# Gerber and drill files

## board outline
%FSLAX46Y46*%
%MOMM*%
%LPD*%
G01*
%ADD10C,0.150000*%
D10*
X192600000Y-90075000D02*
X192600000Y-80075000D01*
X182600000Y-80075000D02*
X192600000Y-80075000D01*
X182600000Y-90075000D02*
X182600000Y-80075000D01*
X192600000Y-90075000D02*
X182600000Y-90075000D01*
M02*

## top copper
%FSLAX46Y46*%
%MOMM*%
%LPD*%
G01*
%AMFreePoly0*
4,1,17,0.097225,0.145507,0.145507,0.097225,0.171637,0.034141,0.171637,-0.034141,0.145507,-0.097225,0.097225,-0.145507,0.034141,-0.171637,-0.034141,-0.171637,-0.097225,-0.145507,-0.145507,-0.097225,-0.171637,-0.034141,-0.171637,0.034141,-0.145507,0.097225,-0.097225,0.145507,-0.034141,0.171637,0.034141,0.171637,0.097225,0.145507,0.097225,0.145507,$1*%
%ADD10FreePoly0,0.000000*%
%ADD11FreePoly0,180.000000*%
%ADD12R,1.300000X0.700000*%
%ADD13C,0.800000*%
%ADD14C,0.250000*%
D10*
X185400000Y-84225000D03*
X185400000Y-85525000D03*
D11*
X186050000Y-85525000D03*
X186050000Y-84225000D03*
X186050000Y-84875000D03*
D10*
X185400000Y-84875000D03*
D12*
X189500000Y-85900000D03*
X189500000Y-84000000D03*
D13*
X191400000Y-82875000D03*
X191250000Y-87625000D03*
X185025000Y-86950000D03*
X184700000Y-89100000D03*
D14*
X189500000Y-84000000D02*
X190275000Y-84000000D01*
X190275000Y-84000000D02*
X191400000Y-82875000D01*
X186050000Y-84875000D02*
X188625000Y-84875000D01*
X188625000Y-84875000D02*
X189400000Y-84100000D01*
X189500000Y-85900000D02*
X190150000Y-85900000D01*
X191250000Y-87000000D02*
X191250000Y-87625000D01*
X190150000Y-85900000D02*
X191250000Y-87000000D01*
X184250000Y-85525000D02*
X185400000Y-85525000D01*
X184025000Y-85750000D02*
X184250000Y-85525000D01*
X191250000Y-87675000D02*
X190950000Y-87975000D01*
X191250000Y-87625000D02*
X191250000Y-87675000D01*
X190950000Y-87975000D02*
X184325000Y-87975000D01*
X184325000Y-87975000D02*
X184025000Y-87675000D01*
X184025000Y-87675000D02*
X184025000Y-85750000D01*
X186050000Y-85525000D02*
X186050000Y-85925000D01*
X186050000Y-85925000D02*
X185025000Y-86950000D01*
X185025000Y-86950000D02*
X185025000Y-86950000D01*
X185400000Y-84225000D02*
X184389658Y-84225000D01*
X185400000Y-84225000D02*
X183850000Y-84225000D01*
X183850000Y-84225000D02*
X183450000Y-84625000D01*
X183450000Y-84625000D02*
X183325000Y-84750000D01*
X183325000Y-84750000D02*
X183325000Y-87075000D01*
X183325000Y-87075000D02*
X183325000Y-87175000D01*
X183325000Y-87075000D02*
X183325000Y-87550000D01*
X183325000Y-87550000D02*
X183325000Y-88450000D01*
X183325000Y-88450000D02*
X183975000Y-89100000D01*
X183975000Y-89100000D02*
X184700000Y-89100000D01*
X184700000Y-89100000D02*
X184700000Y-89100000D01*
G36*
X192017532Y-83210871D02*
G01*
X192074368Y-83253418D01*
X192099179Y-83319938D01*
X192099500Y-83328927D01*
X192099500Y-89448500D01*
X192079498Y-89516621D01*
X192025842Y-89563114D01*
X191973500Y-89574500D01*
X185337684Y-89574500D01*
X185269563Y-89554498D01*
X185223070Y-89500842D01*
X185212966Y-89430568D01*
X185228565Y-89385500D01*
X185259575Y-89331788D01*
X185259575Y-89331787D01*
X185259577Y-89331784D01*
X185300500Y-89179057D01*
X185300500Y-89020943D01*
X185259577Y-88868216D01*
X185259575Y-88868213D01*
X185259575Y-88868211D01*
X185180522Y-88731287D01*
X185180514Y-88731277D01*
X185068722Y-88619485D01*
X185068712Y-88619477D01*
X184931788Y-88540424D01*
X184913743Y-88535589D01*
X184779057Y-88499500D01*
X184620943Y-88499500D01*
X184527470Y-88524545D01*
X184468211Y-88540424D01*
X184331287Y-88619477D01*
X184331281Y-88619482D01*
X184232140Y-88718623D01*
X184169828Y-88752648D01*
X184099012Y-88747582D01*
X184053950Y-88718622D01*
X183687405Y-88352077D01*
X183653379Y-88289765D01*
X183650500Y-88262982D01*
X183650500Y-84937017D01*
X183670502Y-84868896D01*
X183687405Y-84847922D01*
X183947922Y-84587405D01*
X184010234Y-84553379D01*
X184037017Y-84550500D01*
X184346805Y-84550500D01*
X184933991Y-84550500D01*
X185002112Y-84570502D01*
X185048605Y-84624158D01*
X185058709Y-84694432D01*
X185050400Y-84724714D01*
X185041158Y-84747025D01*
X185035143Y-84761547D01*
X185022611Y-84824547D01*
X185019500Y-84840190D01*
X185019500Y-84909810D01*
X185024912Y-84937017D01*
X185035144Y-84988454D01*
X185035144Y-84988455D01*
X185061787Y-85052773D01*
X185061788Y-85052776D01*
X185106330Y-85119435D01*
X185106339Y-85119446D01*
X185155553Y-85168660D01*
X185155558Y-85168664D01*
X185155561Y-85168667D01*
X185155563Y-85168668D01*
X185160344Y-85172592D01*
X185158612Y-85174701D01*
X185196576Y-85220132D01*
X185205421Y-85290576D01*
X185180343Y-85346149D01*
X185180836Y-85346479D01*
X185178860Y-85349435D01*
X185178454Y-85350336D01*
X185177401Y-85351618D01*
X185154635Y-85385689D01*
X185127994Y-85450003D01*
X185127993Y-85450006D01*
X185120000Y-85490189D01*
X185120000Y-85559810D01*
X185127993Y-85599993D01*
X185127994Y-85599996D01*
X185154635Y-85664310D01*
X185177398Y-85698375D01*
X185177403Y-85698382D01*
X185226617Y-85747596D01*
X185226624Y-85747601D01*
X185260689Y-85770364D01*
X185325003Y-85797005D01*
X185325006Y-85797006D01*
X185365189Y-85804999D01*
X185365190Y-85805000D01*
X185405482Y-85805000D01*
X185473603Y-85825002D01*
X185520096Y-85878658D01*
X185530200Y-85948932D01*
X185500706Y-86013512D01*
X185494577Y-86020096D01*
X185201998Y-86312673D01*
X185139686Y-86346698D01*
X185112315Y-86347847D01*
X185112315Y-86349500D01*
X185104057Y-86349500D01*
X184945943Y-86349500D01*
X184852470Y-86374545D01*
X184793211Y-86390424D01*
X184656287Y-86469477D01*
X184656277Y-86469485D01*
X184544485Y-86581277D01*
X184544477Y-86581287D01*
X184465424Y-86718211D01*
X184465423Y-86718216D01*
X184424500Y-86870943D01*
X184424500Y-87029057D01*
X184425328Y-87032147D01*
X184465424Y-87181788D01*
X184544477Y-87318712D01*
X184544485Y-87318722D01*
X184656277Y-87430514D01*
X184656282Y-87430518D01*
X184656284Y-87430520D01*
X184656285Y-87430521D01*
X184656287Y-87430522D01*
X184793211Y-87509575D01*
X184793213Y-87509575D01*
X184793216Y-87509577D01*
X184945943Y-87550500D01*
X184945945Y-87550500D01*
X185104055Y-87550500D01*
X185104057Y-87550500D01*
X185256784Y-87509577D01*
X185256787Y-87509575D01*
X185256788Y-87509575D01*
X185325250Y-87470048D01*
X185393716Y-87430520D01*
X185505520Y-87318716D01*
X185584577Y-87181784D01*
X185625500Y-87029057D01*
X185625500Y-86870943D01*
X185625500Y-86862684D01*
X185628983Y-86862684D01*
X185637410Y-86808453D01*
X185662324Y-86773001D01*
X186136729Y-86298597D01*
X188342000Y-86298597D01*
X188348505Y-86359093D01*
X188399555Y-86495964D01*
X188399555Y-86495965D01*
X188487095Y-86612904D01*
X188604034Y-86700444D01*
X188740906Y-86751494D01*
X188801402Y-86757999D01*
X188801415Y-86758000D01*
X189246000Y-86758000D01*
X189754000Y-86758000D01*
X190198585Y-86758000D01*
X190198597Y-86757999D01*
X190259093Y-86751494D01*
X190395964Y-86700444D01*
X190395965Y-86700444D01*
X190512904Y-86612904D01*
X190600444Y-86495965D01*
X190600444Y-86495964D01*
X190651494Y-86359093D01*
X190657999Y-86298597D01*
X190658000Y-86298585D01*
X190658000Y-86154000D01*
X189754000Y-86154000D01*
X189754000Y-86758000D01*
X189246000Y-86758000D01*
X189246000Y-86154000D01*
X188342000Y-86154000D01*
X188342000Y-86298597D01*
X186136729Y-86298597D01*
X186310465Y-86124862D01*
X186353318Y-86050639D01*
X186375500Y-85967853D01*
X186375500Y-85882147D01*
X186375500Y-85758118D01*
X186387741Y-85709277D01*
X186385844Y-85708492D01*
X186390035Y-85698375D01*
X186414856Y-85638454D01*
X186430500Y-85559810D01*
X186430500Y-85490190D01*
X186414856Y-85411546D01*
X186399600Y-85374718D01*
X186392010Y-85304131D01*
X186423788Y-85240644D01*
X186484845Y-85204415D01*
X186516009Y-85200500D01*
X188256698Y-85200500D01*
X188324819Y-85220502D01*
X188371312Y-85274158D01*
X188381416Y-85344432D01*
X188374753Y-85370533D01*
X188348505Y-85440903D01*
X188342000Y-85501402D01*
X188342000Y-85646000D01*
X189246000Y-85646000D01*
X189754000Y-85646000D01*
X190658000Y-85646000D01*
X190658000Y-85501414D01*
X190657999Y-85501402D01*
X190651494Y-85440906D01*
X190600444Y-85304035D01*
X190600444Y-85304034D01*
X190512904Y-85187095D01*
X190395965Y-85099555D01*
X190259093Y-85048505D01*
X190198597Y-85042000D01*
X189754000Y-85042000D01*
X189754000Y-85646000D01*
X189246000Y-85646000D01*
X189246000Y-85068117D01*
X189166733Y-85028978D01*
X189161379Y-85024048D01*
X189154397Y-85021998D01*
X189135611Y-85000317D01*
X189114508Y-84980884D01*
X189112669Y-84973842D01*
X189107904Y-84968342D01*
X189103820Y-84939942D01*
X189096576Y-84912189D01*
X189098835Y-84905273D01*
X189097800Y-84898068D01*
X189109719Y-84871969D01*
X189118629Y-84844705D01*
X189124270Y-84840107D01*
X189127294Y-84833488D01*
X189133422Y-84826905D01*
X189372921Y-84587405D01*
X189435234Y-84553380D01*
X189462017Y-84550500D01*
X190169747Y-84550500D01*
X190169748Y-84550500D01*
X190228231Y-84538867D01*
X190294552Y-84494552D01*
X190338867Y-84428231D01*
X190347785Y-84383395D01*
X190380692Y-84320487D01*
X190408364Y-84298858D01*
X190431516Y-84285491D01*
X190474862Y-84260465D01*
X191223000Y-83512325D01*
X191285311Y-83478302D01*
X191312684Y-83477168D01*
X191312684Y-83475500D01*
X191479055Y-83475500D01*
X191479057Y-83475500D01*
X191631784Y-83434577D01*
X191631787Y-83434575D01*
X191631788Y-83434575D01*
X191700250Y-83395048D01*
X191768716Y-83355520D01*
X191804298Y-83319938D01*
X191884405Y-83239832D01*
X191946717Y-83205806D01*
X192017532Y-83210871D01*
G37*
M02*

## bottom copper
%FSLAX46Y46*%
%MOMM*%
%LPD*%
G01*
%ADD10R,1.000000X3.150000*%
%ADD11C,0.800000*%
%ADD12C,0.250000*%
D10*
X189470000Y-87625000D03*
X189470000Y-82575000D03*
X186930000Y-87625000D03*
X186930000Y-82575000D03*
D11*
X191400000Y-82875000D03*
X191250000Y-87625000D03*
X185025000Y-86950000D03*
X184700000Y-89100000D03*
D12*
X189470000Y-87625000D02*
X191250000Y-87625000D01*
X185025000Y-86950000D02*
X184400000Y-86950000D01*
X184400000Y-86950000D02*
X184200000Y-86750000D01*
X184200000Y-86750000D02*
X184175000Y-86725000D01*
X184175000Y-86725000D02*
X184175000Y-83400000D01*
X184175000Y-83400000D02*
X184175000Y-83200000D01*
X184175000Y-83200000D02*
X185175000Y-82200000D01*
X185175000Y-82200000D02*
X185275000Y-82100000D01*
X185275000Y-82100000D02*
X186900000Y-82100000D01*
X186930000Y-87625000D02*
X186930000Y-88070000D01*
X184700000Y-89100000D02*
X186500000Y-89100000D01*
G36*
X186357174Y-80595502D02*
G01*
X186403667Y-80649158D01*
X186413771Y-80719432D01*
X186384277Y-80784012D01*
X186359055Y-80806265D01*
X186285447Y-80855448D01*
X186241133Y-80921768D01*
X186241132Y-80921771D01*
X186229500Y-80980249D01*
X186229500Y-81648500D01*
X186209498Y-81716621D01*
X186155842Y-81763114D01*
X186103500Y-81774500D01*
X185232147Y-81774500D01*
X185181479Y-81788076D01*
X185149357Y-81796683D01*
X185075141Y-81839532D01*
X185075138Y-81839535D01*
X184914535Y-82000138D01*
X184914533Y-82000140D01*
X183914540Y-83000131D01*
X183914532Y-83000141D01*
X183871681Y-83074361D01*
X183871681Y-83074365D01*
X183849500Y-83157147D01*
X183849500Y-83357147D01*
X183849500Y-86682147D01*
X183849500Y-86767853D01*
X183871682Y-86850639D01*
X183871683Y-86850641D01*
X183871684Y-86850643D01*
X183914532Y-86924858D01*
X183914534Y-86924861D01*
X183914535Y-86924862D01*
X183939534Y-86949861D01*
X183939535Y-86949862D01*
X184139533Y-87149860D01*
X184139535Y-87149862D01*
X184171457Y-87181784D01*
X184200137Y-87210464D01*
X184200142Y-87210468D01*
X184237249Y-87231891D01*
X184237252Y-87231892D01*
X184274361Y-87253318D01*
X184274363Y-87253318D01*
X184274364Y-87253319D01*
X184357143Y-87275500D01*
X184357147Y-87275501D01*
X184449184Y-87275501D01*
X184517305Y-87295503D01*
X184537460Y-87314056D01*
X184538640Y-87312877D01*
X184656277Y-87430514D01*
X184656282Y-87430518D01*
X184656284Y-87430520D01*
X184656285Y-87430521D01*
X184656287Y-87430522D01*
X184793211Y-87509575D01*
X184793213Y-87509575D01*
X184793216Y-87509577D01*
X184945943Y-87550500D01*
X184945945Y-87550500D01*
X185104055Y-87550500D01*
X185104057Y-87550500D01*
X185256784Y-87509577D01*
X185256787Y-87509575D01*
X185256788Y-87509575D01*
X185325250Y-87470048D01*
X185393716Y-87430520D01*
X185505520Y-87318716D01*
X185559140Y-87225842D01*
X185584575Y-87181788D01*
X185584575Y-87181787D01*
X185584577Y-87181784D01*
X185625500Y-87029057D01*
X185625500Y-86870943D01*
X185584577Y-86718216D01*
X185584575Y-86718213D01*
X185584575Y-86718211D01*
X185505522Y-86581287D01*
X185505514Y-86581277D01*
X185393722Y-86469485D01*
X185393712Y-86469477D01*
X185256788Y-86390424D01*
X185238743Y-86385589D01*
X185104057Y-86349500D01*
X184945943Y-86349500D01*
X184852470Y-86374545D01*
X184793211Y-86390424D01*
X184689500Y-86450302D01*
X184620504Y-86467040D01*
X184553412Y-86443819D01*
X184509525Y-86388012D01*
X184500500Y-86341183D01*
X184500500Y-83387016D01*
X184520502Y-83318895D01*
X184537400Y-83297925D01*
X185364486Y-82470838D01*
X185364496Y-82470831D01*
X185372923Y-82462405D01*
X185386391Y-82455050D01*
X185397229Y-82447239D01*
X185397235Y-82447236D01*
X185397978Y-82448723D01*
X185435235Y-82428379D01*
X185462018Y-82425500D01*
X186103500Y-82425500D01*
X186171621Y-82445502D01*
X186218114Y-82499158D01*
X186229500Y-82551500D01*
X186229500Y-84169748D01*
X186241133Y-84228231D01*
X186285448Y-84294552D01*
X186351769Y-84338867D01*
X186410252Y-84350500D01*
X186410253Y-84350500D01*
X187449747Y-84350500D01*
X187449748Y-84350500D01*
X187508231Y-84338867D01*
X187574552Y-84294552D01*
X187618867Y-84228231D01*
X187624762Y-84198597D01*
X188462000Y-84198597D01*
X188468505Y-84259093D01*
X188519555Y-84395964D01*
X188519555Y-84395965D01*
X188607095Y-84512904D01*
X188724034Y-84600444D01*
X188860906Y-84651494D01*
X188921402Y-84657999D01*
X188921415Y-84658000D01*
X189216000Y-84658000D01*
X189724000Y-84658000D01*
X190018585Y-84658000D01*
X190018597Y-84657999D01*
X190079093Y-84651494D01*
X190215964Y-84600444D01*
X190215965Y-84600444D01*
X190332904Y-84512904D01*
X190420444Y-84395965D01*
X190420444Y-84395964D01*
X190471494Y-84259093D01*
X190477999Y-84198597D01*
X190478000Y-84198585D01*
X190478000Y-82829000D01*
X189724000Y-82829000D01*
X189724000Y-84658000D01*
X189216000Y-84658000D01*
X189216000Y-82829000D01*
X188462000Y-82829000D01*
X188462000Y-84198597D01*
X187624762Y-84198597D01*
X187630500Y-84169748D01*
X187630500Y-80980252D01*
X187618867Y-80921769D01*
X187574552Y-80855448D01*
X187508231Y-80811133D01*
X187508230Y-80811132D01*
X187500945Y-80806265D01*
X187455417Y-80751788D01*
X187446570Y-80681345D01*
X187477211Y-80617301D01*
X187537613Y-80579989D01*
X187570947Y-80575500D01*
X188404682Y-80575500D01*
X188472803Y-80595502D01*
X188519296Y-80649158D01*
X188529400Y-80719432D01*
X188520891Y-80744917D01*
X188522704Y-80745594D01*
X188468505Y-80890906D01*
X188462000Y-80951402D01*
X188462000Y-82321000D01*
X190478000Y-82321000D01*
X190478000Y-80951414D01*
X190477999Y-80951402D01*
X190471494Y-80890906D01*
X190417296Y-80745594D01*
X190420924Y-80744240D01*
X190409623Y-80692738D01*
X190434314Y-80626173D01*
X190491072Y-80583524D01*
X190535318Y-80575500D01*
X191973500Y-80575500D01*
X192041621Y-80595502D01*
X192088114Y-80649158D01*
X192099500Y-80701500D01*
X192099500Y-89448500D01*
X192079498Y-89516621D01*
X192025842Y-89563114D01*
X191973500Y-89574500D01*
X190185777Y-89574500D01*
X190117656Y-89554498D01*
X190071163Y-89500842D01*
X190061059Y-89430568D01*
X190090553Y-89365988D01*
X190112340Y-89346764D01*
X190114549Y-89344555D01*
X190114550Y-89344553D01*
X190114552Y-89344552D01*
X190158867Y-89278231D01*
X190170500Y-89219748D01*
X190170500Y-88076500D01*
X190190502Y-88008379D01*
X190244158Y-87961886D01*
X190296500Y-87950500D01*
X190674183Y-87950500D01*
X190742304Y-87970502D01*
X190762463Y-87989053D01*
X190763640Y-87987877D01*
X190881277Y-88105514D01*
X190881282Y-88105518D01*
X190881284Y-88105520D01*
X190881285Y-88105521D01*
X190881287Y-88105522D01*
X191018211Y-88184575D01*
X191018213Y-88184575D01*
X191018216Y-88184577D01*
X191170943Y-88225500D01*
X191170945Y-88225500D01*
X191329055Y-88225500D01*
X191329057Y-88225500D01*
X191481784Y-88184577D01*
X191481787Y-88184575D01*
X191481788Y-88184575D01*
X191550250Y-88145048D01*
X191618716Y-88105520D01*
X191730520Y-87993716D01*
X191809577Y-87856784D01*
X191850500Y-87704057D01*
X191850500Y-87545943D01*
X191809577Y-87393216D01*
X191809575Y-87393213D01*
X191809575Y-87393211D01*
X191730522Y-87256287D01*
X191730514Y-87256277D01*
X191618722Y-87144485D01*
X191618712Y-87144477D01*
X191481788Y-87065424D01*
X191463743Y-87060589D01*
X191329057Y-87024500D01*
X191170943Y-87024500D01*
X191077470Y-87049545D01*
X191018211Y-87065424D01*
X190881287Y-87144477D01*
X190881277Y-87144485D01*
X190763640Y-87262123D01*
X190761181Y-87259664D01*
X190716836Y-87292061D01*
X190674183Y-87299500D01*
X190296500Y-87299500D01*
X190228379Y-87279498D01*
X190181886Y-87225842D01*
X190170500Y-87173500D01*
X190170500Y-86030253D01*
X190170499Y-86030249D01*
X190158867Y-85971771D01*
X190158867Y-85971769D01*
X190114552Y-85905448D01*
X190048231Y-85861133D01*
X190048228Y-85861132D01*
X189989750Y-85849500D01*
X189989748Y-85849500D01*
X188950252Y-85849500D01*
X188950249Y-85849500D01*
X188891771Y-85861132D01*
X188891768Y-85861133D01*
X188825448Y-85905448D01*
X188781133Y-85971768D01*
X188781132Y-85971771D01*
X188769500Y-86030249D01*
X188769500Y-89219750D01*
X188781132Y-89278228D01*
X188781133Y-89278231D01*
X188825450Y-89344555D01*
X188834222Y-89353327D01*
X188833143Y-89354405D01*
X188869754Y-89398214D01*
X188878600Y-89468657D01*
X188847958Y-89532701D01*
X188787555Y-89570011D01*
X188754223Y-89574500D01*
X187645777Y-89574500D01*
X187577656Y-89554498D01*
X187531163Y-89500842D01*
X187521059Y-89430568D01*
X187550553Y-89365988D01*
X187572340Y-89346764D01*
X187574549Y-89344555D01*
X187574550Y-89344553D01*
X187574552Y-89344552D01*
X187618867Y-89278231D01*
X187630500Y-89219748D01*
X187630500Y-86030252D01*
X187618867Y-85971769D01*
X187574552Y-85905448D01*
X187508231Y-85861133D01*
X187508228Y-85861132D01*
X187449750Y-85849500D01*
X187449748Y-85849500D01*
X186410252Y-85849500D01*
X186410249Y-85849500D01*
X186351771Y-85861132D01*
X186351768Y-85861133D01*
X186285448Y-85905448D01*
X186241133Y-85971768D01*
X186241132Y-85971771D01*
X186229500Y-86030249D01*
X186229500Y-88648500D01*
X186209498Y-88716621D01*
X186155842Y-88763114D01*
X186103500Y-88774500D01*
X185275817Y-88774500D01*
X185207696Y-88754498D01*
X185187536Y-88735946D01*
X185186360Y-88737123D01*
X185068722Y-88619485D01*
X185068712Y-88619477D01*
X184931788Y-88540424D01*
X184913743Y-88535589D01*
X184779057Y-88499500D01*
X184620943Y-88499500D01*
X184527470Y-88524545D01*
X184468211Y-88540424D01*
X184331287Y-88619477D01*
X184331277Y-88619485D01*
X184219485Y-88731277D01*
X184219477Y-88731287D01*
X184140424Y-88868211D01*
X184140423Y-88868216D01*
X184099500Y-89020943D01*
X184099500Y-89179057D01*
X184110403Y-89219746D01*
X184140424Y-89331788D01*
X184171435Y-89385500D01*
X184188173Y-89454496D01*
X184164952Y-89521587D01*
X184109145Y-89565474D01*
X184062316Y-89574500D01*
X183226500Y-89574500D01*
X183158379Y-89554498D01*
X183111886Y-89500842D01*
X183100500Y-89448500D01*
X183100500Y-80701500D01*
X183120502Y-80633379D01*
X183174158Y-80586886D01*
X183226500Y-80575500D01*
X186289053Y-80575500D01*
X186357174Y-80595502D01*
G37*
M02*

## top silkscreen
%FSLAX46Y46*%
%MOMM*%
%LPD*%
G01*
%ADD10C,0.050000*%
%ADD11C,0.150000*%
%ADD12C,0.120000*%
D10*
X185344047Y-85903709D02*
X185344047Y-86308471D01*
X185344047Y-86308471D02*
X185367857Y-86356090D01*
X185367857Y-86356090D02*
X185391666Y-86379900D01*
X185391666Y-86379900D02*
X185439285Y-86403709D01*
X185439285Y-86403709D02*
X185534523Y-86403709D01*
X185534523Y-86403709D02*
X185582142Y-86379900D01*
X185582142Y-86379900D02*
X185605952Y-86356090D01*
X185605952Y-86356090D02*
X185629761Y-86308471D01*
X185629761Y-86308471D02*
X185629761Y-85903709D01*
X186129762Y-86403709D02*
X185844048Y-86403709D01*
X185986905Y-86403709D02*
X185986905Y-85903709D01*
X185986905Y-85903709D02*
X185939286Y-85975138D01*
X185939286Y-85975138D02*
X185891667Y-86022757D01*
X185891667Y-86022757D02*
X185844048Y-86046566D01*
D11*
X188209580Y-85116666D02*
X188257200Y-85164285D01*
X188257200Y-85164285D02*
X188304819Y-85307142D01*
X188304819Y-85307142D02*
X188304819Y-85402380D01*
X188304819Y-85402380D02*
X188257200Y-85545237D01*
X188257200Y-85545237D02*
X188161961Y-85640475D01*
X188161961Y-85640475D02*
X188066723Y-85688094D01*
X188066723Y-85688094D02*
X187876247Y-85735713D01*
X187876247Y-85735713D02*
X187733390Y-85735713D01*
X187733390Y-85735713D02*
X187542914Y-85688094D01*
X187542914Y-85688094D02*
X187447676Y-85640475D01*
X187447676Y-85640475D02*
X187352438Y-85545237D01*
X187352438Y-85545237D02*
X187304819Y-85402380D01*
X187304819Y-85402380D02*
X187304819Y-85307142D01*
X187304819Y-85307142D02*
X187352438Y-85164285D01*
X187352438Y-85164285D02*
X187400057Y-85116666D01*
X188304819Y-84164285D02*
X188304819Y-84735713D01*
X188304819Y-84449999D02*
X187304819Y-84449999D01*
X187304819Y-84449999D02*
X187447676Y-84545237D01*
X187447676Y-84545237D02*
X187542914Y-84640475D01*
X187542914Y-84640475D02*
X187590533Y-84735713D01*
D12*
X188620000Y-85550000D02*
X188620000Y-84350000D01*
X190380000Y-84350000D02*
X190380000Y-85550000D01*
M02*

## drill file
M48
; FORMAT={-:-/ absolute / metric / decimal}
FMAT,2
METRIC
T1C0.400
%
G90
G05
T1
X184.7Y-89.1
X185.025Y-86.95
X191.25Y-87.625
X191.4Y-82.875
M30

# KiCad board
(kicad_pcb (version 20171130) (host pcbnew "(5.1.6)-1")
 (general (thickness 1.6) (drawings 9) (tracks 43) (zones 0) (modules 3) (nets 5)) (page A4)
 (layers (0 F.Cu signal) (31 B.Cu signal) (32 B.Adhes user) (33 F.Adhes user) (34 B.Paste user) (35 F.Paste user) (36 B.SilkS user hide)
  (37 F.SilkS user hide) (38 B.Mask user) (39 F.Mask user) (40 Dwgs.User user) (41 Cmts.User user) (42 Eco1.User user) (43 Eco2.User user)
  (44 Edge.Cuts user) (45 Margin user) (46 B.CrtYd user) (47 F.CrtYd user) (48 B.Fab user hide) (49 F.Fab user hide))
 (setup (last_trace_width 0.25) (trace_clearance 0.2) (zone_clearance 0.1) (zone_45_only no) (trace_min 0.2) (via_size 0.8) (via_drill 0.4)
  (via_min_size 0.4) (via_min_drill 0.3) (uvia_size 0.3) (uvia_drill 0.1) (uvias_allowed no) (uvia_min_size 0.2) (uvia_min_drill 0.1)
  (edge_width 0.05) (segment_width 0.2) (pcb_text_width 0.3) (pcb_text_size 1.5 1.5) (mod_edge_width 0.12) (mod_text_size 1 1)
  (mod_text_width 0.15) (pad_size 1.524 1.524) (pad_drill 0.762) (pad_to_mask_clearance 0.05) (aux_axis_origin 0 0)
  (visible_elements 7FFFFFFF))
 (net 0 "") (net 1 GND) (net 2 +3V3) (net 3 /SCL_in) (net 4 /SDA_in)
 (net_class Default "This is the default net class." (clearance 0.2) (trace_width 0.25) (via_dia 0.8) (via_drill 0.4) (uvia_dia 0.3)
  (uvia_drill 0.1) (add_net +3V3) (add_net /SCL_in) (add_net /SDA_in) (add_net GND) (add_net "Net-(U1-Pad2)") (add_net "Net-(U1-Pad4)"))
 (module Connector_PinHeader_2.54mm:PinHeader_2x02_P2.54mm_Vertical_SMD (layer B.Cu) (at 188.2 85.1 270)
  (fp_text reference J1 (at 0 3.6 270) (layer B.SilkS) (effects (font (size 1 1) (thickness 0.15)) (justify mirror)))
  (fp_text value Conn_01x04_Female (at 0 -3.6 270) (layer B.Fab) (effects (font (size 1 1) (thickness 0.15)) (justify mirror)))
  (pad 4 smd rect (at 2.525 -1.27 270) (size 3.15 1) (layers B.Cu B.Paste B.Mask) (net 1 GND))
  (pad 3 smd rect (at -2.525 -1.27 270) (size 3.15 1) (layers B.Cu B.Paste B.Mask) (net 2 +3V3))
  (pad 2 smd rect (at 2.525 1.27 270) (size 3.15 1) (layers B.Cu B.Paste B.Mask) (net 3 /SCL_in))
  (pad 1 smd rect (at -2.525 1.27 270) (size 3.15 1) (layers B.Cu B.Paste B.Mask) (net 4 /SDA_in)))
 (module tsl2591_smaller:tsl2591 (layer F.Cu) (at 185.725 84.875)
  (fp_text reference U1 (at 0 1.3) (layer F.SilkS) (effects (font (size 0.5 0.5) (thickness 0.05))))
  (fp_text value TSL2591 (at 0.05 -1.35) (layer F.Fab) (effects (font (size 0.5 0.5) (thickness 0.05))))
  (pad 1 smd custom (at -0.325 -0.65) (size 0.35 0.35) (layers F.Cu F.Paste F.Mask) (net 3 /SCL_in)
   (options (clearance outline) (anchor circle)) (primitives))
  (pad 3 smd custom (at -0.325 0.65) (size 0.35 0.35) (layers F.Cu F.Paste F.Mask) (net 1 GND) (zone_connect 0)
   (options (clearance outline) (anchor circle)) (primitives))
  (pad 6 smd custom (at 0.325 0.65 180) (size 0.35 0.35) (layers F.Cu F.Paste F.Mask) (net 4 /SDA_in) (zone_connect 0)
   (options (clearance outline) (anchor circle)) (primitives))
  (pad 4 smd custom (at 0.325 -0.65 180) (size 0.35 0.35) (layers F.Cu F.Paste F.Mask) (zone_connect 0)
   (options (clearance outline) (anchor circle)) (primitives))
  (pad 5 smd custom (at 0.325 0 180) (size 0.35 0.35) (layers F.Cu F.Paste F.Mask) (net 2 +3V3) (zone_connect 0)
   (options (clearance outline) (anchor circle)) (primitives))
  (pad 2 smd custom (at -0.325 0) (size 0.35 0.35) (layers F.Cu F.Paste F.Mask) (options (clearance outline) (anchor circle)) (primitives)))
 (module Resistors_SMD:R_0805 (layer F.Cu) (at 189.5 84.95 90)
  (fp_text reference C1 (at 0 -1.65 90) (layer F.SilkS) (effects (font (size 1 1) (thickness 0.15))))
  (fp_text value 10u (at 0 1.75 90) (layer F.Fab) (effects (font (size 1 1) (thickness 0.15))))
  (fp_line (start -0.6 -0.88) (end 0.6 -0.88) (layer F.SilkS) (width 0.12))
  (fp_line (start 0.6 0.88) (end -0.6 0.88) (layer F.SilkS) (width 0.12))
  (pad 1 smd rect (at -0.95 0 90) (size 0.7 1.3) (layers F.Cu F.Paste F.Mask) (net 1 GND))
  (pad 2 smd rect (at 0.95 0 90) (size 0.7 1.3) (layers F.Cu F.Paste F.Mask) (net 2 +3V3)))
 (gr_line (start 192.6 90.075) (end 192.6 80.075) (layer Edge.Cuts) (width 0.15))
 (gr_line (start 182.6 80.075) (end 192.6 80.075) (layer Edge.Cuts) (width 0.15))
 (gr_line (start 182.6 90.075) (end 182.6 80.075) (layer Edge.Cuts) (width 0.15))
 (gr_line (start 192.6 90.075) (end 182.6 90.075) (layer Edge.Cuts) (width 0.15))
 (segment (start 189.5 84) (end 190.275 84) (width 0.25) (layer F.Cu) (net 2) (status 10))
 (segment (start 190.275 84) (end 191.4 82.875) (width 0.25) (layer F.Cu) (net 2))
 (via (at 191.4 82.875) (size 0.8) (drill 0.4) (layers F.Cu B.Cu) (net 2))
 (segment (start 186.05 84.875) (end 188.625 84.875) (width 0.25) (layer F.Cu) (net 2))
 (segment (start 188.625 84.875) (end 189.4 84.1) (width 0.25) (layer F.Cu) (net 2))
 (segment (start 189.47 87.625) (end 191.25 87.625) (width 0.25) (layer B.Cu) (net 1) (status 10))
 (via (at 191.25 87.625) (size 0.8) (drill 0.4) (layers F.Cu B.Cu) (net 1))
 (segment (start 189.5 85.9) (end 190.15 85.9) (width 0.25) (layer F.Cu) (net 1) (status 30))
 (segment (start 191.25 87) (end 191.25 87.625) (width 0.25) (layer F.Cu) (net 1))
 (segment (start 190.15 85.9) (end 191.25 87) (width 0.25) (layer F.Cu) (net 1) (status 10))
 (segment (start 184.25 85.525) (end 185.4 85.525) (width 0.25) (layer F.Cu) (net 1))
 (segment (start 184.025 85.75) (end 184.25 85.525) (width 0.25) (layer F.Cu) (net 1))
 (segment (start 191.25 87.675) (end 190.95 87.975) (width 0.25) (layer F.Cu) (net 1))
 (segment (start 191.25 87.625) (end 191.25 87.675) (width 0.25) (layer F.Cu) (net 1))
 (segment (start 190.95 87.975) (end 184.325 87.975) (width 0.25) (layer F.Cu) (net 1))
 (segment (start 184.325 87.975) (end 184.025 87.675) (width 0.25) (layer F.Cu) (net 1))
 (segment (start 184.025 87.675) (end 184.025 85.75) (width 0.25) (layer F.Cu) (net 1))
 (segment (start 186.05 85.525) (end 186.05 85.925) (width 0.25) (layer F.Cu) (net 4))
 (segment (start 186.05 85.925) (end 185.025 86.95) (width 0.25) (layer F.Cu) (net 4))
 (segment (start 185.025 86.95) (end 185.025 86.95) (width 0.25) (layer F.Cu) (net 4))
 (via (at 185.025 86.95) (size 0.8) (drill 0.4) (layers F.Cu B.Cu) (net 4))
 (segment (start 185.025 86.95) (end 184.4 86.95) (width 0.25) (layer B.Cu) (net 4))
 (segment (start 184.4 86.95) (end 184.2 86.75) (width 0.25) (layer B.Cu) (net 4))
 (segment (start 184.2 86.75) (end 184.175 86.725) (width 0.25) (layer B.Cu) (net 4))
 (segment (start 184.175 86.725) (end 184.175 83.4) (width 0.25) (layer B.Cu) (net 4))
 (segment (start 184.175 83.4) (end 184.175 83.2) (width 0.25) (layer B.Cu) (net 4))
 (segment (start 184.175 83.2) (end 185.175 82.2) (width 0.25) (layer B.Cu) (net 4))
 (segment (start 185.175 82.2) (end 185.275 82.1) (width 0.25) (layer B.Cu) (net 4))
 (segment (start 185.275 82.1) (end 186.9 82.1) (width 0.25) (layer B.Cu) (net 4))
 (segment (start 186.93 87.625) (end 186.93 88.07) (width 0.25) (layer B.Cu) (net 3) (status 30))
 (segment (start 185.4 84.225) (end 184.389658 84.225) (width 0.25) (layer F.Cu) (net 3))
 (segment (start 185.4 84.225) (end 183.85 84.225) (width 0.25) (layer F.Cu) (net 3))
 (segment (start 183.85 84.225) (end 183.45 84.625) (width 0.25) (layer F.Cu) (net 3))
 (segment (start 183.45 84.625) (end 183.325 84.75) (width 0.25) (layer F.Cu) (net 3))
 (segment (start 183.325 84.75) (end 183.325 87.075) (width 0.25) (layer F.Cu) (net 3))
 (segment (start 183.325 87.075) (end 183.325 87.175) (width 0.25) (layer F.Cu) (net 3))
 (segment (start 183.325 87.075) (end 183.325 87.55) (width 0.25) (layer F.Cu) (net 3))
 (segment (start 183.325 87.55) (end 183.325 88.45) (width 0.25) (layer F.Cu) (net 3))
 (segment (start 183.325 88.45) (end 183.975 89.1) (width 0.25) (layer F.Cu) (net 3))
 (segment (start 183.975 89.1) (end 184.7 89.1) (width 0.25) (layer F.Cu) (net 3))
 (segment (start 184.7 89.1) (end 184.7 89.1) (width 0.25) (layer F.Cu) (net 3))
 (via (at 184.7 89.1) (size 0.8) (drill 0.4) (layers F.Cu B.Cu) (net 3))
 (segment (start 184.7 89.1) (end 186.5 89.1) (width 0.25) (layer B.Cu) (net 3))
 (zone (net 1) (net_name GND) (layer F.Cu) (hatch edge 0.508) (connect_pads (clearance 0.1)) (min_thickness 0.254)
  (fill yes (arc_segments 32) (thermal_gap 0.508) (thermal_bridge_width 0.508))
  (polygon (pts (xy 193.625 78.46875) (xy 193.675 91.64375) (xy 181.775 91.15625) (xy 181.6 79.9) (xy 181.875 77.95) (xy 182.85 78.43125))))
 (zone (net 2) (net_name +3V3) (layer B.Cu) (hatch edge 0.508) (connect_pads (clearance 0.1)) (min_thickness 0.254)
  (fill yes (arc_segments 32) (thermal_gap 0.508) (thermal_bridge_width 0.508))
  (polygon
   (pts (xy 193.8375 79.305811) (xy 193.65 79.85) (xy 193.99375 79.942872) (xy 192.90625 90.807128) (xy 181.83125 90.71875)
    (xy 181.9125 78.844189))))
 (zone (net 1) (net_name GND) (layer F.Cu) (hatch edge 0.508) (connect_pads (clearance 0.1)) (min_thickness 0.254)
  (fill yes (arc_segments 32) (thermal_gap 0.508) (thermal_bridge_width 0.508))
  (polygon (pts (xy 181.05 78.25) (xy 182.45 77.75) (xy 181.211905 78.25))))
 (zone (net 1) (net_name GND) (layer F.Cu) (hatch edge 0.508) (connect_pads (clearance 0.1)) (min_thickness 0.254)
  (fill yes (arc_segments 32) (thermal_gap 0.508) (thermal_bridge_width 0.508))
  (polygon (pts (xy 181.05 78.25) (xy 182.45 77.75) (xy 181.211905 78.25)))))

